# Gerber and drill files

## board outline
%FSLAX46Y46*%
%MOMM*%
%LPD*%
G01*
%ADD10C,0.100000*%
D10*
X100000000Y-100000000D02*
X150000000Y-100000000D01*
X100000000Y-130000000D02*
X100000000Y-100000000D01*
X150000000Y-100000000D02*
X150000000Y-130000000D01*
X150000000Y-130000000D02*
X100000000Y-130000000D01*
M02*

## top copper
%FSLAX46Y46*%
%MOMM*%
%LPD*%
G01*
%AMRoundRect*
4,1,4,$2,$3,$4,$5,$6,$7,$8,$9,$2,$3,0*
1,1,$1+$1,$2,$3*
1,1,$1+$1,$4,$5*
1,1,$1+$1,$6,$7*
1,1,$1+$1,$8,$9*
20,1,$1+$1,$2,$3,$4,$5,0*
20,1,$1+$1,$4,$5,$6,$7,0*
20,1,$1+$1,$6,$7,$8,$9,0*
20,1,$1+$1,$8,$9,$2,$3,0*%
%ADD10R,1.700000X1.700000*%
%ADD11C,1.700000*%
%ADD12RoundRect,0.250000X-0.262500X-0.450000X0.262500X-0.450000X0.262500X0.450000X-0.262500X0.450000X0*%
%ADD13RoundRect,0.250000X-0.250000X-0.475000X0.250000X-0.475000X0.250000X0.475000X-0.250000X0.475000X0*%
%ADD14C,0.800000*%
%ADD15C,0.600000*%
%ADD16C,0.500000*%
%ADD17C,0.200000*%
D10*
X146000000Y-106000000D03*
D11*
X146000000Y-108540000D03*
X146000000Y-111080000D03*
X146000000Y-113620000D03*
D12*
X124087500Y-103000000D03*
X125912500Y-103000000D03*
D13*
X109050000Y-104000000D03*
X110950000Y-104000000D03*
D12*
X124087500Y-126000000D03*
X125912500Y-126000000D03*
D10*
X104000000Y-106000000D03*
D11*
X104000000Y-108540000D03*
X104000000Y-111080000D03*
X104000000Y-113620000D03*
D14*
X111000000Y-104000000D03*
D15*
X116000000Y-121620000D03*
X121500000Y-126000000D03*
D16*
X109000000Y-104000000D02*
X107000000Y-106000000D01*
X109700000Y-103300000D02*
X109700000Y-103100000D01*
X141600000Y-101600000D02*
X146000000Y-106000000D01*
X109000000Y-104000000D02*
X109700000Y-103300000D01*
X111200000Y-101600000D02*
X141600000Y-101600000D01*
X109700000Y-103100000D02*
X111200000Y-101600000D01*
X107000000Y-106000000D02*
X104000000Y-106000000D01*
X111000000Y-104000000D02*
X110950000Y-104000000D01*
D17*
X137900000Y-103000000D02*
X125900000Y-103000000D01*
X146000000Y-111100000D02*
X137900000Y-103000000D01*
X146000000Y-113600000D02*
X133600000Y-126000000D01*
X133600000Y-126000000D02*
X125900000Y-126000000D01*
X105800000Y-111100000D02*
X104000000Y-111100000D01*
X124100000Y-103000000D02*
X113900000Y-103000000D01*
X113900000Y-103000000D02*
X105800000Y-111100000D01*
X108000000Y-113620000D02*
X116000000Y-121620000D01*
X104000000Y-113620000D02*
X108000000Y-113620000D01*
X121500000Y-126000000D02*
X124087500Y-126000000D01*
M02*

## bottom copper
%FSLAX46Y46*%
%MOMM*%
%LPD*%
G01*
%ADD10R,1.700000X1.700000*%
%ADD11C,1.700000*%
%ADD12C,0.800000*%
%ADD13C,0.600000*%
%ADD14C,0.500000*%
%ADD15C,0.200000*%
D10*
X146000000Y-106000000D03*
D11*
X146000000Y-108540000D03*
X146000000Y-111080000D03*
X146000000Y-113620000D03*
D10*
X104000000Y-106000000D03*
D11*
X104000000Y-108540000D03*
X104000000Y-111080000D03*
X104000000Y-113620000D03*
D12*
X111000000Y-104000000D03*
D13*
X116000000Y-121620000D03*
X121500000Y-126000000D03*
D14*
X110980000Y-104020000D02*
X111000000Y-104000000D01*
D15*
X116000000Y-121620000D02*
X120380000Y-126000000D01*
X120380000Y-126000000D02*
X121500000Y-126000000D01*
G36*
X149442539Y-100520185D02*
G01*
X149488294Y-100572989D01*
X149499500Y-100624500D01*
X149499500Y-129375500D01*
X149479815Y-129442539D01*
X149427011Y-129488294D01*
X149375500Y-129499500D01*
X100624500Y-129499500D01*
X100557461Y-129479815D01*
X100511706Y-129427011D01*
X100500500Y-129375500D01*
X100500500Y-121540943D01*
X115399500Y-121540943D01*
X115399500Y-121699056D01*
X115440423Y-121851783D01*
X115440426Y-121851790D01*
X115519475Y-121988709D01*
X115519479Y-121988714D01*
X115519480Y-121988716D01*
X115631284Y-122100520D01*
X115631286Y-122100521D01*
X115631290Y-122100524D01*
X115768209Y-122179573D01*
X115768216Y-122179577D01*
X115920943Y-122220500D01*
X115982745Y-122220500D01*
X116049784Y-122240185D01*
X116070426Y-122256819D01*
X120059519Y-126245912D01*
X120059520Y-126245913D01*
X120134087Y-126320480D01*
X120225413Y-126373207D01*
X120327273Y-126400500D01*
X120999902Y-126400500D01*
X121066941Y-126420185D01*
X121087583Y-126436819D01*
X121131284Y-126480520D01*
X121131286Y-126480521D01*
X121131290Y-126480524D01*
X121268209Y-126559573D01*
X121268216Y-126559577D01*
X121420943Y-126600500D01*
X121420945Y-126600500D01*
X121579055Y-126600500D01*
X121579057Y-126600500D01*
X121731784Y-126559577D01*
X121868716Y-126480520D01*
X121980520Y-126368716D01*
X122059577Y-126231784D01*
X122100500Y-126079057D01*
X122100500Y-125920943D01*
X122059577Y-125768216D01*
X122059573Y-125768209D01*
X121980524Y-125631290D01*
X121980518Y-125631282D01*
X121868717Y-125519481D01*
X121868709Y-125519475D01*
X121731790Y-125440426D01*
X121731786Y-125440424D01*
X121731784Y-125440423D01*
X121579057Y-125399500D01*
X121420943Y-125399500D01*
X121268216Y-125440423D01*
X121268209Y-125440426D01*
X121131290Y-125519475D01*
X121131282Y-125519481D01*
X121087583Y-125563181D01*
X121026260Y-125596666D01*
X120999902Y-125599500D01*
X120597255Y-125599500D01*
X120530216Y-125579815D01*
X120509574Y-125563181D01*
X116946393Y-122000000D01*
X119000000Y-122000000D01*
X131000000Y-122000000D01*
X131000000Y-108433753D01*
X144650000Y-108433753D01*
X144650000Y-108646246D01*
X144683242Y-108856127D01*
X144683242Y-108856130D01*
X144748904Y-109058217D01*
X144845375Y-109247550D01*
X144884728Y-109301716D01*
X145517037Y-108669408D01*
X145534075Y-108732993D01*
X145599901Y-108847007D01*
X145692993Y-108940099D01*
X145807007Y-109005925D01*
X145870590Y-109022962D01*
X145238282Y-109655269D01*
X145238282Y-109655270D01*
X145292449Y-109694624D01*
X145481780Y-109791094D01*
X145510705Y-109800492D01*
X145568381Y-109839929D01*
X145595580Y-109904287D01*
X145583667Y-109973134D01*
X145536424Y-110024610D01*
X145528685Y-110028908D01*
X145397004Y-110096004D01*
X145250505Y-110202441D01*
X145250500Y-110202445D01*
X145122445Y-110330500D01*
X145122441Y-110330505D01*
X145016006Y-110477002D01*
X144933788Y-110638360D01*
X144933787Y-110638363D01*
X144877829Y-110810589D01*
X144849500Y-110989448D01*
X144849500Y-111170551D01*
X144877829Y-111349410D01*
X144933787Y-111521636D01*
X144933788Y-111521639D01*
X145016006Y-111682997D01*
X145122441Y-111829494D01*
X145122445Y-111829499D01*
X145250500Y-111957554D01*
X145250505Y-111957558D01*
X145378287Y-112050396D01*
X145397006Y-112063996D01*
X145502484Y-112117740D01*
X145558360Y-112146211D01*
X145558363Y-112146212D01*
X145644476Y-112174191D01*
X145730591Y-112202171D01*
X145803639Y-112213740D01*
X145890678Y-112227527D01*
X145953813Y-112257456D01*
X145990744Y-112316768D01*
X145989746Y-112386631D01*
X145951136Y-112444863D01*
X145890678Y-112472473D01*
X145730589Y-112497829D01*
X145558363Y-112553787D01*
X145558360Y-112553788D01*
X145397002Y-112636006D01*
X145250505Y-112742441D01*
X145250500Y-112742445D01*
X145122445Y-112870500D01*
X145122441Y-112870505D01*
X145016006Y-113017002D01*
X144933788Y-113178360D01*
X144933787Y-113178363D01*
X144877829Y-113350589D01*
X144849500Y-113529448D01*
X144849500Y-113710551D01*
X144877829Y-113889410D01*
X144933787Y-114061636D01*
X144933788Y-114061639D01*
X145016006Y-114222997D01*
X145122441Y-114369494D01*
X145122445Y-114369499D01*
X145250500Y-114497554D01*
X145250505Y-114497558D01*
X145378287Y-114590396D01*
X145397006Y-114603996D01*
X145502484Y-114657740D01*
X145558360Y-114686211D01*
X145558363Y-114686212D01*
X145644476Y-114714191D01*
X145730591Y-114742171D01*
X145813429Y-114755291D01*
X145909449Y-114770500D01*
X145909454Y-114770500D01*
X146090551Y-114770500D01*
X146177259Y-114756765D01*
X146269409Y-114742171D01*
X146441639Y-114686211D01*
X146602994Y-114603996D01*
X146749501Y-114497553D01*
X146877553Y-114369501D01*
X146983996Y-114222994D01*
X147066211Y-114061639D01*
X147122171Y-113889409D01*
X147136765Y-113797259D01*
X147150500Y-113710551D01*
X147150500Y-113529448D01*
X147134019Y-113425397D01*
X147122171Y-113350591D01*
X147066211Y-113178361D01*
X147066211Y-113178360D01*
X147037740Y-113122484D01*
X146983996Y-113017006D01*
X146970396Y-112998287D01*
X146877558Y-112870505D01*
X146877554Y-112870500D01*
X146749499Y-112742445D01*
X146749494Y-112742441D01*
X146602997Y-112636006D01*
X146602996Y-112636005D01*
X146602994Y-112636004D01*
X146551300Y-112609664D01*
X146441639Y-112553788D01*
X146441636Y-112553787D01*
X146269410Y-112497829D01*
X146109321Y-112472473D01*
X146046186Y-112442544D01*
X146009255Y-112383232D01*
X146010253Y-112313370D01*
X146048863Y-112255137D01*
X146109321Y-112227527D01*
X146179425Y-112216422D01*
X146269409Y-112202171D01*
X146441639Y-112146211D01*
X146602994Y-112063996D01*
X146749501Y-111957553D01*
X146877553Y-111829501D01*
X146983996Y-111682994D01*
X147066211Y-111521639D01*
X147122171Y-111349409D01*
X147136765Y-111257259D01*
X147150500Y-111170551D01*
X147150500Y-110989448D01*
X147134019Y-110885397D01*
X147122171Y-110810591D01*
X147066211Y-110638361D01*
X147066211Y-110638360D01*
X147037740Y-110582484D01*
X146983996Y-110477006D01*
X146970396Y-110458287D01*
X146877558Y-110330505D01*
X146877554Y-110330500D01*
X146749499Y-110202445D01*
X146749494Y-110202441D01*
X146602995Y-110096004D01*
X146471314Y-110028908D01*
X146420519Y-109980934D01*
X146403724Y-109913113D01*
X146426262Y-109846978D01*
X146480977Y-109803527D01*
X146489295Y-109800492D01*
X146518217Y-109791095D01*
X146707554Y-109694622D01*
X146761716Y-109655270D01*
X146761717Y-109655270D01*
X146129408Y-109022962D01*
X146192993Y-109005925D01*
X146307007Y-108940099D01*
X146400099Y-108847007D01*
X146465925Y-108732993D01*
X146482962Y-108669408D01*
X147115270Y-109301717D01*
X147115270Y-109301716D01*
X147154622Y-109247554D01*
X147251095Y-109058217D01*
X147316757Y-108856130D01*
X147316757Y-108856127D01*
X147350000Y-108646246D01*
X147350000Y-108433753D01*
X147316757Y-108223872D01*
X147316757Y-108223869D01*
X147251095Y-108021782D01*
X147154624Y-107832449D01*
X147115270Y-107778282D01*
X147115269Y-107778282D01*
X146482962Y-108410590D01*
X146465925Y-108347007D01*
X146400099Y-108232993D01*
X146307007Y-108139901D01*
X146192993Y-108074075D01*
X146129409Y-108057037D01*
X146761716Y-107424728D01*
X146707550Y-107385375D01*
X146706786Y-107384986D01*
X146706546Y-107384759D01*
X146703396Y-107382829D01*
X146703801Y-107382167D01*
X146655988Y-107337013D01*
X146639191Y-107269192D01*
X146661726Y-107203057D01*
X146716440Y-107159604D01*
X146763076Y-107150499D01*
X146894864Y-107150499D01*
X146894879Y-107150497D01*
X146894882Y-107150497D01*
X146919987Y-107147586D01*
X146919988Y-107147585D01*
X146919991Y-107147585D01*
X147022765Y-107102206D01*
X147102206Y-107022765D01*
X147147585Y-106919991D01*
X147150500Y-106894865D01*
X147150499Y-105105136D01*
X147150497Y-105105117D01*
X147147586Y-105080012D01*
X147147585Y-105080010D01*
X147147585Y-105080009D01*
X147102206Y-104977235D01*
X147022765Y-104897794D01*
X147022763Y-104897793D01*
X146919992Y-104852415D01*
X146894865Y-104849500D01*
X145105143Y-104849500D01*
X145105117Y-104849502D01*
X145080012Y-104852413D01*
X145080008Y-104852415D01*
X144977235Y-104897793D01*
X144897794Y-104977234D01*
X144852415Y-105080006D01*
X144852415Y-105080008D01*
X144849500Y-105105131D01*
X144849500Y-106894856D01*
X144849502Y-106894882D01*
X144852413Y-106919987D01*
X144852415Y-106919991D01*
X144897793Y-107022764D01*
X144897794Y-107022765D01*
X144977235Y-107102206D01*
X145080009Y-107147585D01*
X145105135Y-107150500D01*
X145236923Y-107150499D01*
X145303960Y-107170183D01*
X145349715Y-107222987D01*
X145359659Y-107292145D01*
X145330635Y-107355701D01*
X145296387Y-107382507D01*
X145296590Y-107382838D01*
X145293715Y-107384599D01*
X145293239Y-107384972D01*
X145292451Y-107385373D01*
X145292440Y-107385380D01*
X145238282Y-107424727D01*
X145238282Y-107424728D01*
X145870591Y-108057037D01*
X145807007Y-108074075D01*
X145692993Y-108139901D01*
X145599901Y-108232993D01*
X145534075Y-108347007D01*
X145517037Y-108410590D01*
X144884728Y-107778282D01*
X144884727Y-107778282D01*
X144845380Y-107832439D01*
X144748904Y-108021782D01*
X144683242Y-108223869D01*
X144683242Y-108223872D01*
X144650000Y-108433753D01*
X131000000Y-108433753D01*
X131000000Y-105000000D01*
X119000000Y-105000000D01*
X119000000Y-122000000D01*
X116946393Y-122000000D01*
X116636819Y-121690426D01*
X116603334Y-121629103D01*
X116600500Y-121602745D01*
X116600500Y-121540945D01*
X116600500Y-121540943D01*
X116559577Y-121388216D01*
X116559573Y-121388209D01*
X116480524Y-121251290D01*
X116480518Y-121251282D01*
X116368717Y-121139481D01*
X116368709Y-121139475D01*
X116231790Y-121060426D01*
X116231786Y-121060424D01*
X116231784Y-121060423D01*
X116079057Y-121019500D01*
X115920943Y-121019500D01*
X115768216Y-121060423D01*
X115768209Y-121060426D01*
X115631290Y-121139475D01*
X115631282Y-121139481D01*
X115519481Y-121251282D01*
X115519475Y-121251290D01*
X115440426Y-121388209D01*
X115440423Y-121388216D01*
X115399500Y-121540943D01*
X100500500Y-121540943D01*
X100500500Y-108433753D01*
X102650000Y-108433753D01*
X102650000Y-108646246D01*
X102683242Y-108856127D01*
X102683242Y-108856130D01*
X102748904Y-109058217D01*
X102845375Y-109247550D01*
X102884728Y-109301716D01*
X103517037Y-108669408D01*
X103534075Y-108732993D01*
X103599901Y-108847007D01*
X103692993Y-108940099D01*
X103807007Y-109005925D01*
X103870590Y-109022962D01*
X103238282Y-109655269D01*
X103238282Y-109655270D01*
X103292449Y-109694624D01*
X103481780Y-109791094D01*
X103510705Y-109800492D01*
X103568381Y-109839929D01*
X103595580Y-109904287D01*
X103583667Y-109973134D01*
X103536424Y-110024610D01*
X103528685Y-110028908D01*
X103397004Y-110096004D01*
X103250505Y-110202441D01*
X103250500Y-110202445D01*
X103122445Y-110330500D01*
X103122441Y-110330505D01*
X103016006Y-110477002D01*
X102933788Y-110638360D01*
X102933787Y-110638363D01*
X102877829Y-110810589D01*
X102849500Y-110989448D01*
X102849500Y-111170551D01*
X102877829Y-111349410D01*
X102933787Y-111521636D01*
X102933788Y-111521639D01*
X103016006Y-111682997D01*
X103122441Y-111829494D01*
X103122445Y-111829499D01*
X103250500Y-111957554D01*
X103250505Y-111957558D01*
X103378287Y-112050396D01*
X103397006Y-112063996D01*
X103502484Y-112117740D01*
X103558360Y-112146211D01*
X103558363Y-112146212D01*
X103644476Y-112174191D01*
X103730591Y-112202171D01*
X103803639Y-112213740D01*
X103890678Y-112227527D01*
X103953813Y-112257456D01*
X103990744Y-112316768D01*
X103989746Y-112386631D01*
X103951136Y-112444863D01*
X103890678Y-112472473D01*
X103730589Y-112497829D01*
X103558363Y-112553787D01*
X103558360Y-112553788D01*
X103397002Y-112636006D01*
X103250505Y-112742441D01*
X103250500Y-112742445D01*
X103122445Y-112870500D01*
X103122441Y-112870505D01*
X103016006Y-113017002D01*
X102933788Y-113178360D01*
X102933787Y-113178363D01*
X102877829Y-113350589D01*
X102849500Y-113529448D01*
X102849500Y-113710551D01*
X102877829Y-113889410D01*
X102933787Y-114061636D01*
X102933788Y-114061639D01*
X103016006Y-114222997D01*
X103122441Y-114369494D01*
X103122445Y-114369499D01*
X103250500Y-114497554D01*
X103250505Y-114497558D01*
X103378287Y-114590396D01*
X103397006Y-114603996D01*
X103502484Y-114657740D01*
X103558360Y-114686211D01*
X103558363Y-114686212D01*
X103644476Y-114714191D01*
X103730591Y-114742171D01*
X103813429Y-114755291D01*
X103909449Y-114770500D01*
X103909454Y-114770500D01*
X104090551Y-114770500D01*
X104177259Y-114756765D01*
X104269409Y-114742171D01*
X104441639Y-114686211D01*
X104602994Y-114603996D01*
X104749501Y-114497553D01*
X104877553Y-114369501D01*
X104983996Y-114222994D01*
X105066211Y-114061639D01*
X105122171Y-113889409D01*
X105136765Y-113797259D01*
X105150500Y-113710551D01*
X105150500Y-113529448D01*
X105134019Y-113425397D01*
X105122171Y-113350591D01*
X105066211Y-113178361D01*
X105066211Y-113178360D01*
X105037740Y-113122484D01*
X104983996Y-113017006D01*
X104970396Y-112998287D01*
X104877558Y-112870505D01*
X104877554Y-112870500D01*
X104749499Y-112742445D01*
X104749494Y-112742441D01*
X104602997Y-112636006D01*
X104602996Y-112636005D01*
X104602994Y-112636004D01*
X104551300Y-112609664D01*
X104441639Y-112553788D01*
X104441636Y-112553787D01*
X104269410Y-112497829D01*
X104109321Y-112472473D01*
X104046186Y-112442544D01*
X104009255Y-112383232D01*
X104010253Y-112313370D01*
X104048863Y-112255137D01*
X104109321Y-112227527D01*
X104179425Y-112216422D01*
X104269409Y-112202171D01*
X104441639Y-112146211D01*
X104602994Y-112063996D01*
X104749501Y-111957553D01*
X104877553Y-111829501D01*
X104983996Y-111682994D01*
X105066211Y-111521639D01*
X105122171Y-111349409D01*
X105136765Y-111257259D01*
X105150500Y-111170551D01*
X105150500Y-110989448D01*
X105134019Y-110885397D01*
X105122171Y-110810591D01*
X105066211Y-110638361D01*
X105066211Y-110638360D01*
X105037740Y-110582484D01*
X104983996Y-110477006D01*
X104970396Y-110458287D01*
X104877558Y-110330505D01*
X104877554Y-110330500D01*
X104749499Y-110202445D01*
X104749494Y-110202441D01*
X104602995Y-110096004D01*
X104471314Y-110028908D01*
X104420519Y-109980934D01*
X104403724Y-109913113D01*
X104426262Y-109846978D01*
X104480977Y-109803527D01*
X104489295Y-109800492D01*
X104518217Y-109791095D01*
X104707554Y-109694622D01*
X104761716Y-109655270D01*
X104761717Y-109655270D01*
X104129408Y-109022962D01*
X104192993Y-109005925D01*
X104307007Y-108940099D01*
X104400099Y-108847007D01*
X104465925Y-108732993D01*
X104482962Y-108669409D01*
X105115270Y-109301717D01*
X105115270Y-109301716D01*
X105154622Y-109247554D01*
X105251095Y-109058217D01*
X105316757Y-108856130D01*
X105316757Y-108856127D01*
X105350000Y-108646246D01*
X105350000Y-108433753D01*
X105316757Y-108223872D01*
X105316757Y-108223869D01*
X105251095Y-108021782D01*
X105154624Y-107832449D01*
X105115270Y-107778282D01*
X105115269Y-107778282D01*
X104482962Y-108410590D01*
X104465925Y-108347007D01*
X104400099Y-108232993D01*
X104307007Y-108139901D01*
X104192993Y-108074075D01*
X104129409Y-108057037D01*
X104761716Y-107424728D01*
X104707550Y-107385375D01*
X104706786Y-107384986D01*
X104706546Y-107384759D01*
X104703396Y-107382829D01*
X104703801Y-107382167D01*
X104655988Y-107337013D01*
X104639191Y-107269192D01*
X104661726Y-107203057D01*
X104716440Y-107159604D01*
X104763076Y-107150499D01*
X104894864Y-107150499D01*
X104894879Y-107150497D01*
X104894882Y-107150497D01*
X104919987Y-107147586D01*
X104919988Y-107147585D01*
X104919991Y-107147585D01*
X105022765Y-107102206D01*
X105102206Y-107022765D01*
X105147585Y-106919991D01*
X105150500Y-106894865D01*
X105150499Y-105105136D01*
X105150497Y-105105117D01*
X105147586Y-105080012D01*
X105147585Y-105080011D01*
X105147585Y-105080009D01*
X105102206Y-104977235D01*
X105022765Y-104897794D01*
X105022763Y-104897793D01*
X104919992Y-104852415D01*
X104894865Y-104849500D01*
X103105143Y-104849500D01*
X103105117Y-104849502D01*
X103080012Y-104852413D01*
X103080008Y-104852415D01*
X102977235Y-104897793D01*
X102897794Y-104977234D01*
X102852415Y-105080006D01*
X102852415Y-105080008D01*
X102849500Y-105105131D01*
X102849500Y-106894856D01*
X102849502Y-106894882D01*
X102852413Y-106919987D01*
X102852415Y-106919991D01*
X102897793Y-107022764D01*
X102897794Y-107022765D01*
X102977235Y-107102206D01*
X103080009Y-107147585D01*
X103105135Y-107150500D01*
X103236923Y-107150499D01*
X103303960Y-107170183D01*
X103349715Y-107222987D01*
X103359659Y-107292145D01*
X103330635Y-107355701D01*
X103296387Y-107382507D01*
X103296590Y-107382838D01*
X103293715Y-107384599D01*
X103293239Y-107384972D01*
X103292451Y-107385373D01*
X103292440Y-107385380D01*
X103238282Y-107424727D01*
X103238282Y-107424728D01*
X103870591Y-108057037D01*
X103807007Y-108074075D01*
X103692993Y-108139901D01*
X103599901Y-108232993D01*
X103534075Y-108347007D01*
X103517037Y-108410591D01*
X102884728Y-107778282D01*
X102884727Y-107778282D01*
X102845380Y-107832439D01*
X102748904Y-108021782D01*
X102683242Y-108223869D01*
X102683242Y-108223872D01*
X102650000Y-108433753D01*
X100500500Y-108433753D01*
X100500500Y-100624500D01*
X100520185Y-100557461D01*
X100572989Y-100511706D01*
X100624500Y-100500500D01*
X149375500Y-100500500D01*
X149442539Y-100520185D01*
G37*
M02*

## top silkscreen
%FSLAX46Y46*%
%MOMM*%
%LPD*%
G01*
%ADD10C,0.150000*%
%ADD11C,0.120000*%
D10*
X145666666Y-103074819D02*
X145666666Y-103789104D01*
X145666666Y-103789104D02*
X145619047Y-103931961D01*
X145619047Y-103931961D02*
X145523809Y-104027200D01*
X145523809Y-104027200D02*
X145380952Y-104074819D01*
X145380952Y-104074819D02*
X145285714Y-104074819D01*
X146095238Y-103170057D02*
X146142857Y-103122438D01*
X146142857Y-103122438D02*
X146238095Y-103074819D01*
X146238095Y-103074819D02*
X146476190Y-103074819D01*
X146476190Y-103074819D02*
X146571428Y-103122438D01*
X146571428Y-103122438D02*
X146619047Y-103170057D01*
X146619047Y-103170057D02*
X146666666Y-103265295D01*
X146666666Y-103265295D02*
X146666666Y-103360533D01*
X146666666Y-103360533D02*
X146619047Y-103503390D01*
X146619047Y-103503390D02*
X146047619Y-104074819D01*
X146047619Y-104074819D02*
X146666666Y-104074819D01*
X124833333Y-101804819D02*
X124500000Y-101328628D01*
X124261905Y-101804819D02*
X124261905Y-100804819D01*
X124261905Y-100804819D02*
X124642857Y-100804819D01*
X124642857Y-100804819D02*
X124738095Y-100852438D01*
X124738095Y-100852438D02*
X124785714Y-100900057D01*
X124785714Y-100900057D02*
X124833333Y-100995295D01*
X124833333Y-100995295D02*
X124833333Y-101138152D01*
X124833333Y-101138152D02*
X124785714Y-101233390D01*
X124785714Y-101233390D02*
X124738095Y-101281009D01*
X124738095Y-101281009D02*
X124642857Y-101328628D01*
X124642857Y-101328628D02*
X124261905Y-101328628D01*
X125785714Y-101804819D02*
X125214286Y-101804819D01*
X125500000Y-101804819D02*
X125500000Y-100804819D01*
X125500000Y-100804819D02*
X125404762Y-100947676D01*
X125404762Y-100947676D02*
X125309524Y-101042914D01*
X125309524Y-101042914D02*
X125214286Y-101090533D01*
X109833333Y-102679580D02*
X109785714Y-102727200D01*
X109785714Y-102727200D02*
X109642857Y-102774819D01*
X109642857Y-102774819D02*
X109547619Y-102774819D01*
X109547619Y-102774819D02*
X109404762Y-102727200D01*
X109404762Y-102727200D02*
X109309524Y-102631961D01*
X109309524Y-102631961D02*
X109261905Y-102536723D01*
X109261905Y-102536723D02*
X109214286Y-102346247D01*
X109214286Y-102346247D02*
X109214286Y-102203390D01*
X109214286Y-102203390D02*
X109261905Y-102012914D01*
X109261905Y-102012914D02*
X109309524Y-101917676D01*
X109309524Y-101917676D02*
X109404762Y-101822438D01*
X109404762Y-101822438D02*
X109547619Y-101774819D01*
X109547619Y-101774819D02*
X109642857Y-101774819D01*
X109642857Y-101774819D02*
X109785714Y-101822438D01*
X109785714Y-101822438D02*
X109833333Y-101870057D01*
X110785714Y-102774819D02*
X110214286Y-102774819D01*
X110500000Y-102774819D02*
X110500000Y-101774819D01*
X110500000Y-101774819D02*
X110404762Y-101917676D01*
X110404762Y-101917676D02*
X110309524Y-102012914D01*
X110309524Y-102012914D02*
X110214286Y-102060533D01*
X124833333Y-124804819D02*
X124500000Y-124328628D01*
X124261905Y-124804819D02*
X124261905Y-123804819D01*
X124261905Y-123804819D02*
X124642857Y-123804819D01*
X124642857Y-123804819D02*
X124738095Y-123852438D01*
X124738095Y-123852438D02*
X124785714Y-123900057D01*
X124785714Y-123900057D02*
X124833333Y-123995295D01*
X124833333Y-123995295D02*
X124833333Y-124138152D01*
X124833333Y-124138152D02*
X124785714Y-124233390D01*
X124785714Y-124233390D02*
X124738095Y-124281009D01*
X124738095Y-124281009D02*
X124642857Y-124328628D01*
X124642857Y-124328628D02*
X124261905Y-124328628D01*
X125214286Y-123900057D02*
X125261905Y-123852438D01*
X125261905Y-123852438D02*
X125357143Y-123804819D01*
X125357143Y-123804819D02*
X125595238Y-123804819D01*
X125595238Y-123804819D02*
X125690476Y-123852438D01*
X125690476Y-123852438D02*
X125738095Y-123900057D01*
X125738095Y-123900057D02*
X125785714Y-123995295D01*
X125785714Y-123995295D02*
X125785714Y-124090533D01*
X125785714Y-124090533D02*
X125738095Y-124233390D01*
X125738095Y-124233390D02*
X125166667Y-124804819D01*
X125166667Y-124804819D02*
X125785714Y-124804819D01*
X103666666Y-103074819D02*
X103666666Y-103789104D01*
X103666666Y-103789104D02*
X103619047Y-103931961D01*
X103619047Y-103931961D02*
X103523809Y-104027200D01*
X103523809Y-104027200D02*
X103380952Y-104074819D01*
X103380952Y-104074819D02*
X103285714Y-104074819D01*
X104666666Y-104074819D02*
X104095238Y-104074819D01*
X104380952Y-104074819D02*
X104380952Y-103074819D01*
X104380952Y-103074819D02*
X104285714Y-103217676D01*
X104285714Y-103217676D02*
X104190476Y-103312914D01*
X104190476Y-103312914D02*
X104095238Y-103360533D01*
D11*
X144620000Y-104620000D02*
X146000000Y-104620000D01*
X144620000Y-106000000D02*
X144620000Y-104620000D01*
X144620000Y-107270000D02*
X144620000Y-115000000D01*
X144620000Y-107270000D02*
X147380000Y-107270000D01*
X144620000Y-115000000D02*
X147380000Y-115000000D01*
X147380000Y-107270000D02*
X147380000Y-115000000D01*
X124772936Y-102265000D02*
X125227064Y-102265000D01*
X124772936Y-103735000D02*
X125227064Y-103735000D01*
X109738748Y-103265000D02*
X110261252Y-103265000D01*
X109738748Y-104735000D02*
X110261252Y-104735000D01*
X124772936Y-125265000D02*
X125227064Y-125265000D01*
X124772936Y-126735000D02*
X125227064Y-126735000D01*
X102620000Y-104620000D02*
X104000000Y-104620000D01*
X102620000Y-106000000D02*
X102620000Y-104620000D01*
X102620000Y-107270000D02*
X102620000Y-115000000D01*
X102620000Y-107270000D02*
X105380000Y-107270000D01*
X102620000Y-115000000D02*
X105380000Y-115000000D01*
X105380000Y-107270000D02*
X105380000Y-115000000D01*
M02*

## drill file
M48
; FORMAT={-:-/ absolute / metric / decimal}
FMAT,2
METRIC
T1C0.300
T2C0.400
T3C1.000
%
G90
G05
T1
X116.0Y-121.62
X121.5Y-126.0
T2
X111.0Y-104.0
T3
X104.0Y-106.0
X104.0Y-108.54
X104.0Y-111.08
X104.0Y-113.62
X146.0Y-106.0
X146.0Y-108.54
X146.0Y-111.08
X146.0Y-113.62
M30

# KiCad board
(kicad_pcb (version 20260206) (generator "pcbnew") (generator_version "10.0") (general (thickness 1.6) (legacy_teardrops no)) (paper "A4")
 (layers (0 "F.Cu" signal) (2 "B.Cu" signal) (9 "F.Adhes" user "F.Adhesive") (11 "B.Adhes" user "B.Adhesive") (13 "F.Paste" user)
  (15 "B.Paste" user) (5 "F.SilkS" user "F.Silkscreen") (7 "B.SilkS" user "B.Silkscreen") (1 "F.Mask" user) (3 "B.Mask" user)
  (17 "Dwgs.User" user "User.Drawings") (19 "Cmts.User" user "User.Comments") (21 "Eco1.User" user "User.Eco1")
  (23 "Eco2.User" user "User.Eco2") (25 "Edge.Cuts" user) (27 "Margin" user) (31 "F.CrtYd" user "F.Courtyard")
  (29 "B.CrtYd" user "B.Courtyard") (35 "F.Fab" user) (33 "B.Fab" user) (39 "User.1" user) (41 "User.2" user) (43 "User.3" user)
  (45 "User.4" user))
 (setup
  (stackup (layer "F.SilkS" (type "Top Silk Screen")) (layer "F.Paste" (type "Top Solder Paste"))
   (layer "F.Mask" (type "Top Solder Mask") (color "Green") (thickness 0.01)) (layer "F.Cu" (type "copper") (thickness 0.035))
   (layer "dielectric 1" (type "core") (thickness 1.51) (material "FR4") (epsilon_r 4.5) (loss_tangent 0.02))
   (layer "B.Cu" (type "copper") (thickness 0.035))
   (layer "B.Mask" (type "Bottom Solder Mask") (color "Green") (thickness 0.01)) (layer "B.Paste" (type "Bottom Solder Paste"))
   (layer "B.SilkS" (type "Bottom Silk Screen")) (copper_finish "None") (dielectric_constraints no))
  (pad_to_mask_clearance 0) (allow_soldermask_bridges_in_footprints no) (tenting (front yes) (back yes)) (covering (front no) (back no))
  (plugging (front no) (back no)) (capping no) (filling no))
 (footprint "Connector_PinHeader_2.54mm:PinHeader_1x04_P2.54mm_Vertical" (layer "F.Cu") (at 146 106)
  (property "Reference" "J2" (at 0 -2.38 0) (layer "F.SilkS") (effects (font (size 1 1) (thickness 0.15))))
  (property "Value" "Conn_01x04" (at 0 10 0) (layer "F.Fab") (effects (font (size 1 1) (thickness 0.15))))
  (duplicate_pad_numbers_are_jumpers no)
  (fp_line (start -1.38 -1.38) (end 0 -1.38) (stroke (width 0.12) (type solid)) (layer "F.SilkS"))
  (fp_line (start -1.38 0) (end -1.38 -1.38) (stroke (width 0.12) (type solid)) (layer "F.SilkS"))
  (fp_line (start -1.38 1.27) (end -1.38 9) (stroke (width 0.12) (type solid)) (layer "F.SilkS"))
  (fp_line (start -1.38 1.27) (end 1.38 1.27) (stroke (width 0.12) (type solid)) (layer "F.SilkS"))
  (fp_line (start -1.38 9) (end 1.38 9) (stroke (width 0.12) (type solid)) (layer "F.SilkS"))
  (fp_line (start 1.38 1.27) (end 1.38 9) (stroke (width 0.12) (type solid)) (layer "F.SilkS"))
  (pad "1" thru_hole rect (at 0 0) (size 1.7 1.7) (drill 1) (layers "*.Cu" "*.Mask") (remove_unused_layers no) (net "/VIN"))
  (pad "2" thru_hole circle (at 0 2.54) (size 1.7 1.7) (drill 1) (layers "*.Cu" "*.Mask") (remove_unused_layers no) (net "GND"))
  (pad "3" thru_hole circle (at 0 5.08) (size 1.7 1.7) (drill 1) (layers "*.Cu" "*.Mask") (remove_unused_layers no) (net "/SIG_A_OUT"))
  (pad "4" thru_hole circle (at 0 7.62) (size 1.7 1.7) (drill 1) (layers "*.Cu" "*.Mask") (remove_unused_layers no) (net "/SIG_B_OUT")))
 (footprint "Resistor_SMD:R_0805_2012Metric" (layer "F.Cu") (at 125 103)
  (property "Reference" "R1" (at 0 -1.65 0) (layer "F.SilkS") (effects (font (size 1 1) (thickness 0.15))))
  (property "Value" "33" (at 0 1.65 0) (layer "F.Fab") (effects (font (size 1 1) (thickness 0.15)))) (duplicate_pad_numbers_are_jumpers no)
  (fp_line (start -0.227064 -0.735) (end 0.227064 -0.735) (stroke (width 0.12) (type solid)) (layer "F.SilkS"))
  (fp_line (start -0.227064 0.735) (end 0.227064 0.735) (stroke (width 0.12) (type solid)) (layer "F.SilkS"))
  (pad "1" smd roundrect (at -0.9125 0) (size 1.025 1.4) (layers "F.Cu" "F.Mask" "F.Paste") (roundrect_rratio 0.243902) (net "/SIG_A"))
  (pad "2" smd roundrect (at 0.9125 0) (size 1.025 1.4) (layers "F.Cu" "F.Mask" "F.Paste") (roundrect_rratio 0.243902) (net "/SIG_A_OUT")))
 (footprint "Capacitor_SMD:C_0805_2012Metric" (layer "F.Cu") (at 110 104)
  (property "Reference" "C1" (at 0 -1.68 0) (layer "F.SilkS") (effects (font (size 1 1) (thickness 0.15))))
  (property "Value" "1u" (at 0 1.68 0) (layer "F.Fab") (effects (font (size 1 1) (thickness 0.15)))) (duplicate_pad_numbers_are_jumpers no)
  (fp_line (start -0.261252 -0.735) (end 0.261252 -0.735) (stroke (width 0.12) (type solid)) (layer "F.SilkS"))
  (fp_line (start -0.261252 0.735) (end 0.261252 0.735) (stroke (width 0.12) (type solid)) (layer "F.SilkS"))
  (pad "1" smd roundrect (at -0.95 0) (size 1 1.45) (layers "F.Cu" "F.Mask" "F.Paste") (roundrect_rratio 0.25) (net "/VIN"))
  (pad "2" smd roundrect (at 0.95 0) (size 1 1.45) (layers "F.Cu" "F.Mask" "F.Paste") (roundrect_rratio 0.25) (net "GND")))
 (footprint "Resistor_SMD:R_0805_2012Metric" (layer "F.Cu") (at 125 126)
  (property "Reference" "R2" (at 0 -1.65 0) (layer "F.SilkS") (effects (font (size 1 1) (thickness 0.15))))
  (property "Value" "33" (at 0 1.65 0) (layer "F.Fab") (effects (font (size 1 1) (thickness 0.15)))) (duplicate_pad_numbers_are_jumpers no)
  (fp_line (start -0.227064 -0.735) (end 0.227064 -0.735) (stroke (width 0.12) (type solid)) (layer "F.SilkS"))
  (fp_line (start -0.227064 0.735) (end 0.227064 0.735) (stroke (width 0.12) (type solid)) (layer "F.SilkS"))
  (pad "1" smd roundrect (at -0.9125 0) (size 1.025 1.4) (layers "F.Cu" "F.Mask" "F.Paste") (roundrect_rratio 0.243902) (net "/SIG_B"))
  (pad "2" smd roundrect (at 0.9125 0) (size 1.025 1.4) (layers "F.Cu" "F.Mask" "F.Paste") (roundrect_rratio 0.243902) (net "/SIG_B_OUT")))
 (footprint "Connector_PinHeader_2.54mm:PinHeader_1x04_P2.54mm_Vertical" (layer "F.Cu") (at 104 106)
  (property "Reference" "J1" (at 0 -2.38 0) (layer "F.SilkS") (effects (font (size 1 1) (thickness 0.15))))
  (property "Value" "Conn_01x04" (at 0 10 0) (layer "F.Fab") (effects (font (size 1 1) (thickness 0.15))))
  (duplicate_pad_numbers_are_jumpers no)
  (fp_line (start -1.38 -1.38) (end 0 -1.38) (stroke (width 0.12) (type solid)) (layer "F.SilkS"))
  (fp_line (start -1.38 0) (end -1.38 -1.38) (stroke (width 0.12) (type solid)) (layer "F.SilkS"))
  (fp_line (start -1.38 1.27) (end -1.38 9) (stroke (width 0.12) (type solid)) (layer "F.SilkS"))
  (fp_line (start -1.38 1.27) (end 1.38 1.27) (stroke (width 0.12) (type solid)) (layer "F.SilkS"))
  (fp_line (start -1.38 9) (end 1.38 9) (stroke (width 0.12) (type solid)) (layer "F.SilkS"))
  (fp_line (start 1.38 1.27) (end 1.38 9) (stroke (width 0.12) (type solid)) (layer "F.SilkS"))
  (pad "1" thru_hole rect (at 0 0) (size 1.7 1.7) (drill 1) (layers "*.Cu" "*.Mask") (remove_unused_layers no) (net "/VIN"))
  (pad "2" thru_hole circle (at 0 2.54) (size 1.7 1.7) (drill 1) (layers "*.Cu" "*.Mask") (remove_unused_layers no) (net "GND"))
  (pad "3" thru_hole circle (at 0 5.08) (size 1.7 1.7) (drill 1) (layers "*.Cu" "*.Mask") (remove_unused_layers no) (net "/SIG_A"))
  (pad "4" thru_hole circle (at 0 7.62) (size 1.7 1.7) (drill 1) (layers "*.Cu" "*.Mask") (remove_unused_layers no) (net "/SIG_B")))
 (gr_line (start 100 100) (end 150 100) (stroke (width 0.1) (type default)) (layer "Edge.Cuts"))
 (gr_line (start 100 130) (end 100 100) (stroke (width 0.1) (type default)) (layer "Edge.Cuts"))
 (gr_line (start 150 100) (end 150 130) (stroke (width 0.1) (type default)) (layer "Edge.Cuts"))
 (gr_line (start 150 130) (end 100 130) (stroke (width 0.1) (type default)) (layer "Edge.Cuts"))
 (segment (start 109 104) (end 107 106) (width 0.5) (layer "F.Cu") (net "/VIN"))
 (segment (start 109.7 103.3) (end 109.7 103.1) (width 0.5) (layer "F.Cu") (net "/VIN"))
 (segment (start 141.6 101.6) (end 146 106) (width 0.5) (layer "F.Cu") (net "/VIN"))
 (segment (start 109 104) (end 109.7 103.3) (width 0.5) (layer "F.Cu") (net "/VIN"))
 (segment (start 111.2 101.6) (end 141.6 101.6) (width 0.5) (layer "F.Cu") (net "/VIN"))
 (segment (start 109.7 103.1) (end 111.2 101.6) (width 0.5) (layer "F.Cu") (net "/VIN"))
 (segment (start 107 106) (end 104 106) (width 0.5) (layer "F.Cu") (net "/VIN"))
 (segment (start 111 104) (end 110.95 104) (width 0.5) (layer "F.Cu") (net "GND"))
 (via (at 111 104) (size 0.8) (drill 0.4) (layers "F.Cu" "B.Cu") (capping yes) (filling yes) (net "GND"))
 (segment (start 110.98 104.02) (end 111 104) (width 0.5) (layer "B.Cu") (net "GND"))
 (segment (start 137.9 103) (end 125.9 103) (width 0.2) (layer "F.Cu") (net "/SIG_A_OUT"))
 (segment (start 146 111.1) (end 137.9 103) (width 0.2) (layer "F.Cu") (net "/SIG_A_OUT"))
 (segment (start 146 113.6) (end 133.6 126) (width 0.2) (layer "F.Cu") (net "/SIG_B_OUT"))
 (segment (start 133.6 126) (end 125.9 126) (width 0.2) (layer "F.Cu") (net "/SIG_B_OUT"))
 (segment (start 105.8 111.1) (end 104 111.1) (width 0.2) (layer "F.Cu") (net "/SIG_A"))
 (segment (start 124.1 103) (end 113.9 103) (width 0.2) (layer "F.Cu") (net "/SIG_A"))
 (segment (start 113.9 103) (end 105.8 111.1) (width 0.2) (layer "F.Cu") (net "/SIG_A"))
 (segment (start 108 113.62) (end 116 121.62) (width 0.2) (locked yes) (layer "F.Cu") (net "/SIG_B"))
 (segment (start 104 113.62) (end 108 113.62) (width 0.2) (locked yes) (layer "F.Cu") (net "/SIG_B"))
 (segment (start 121.5 126) (end 124.0875 126) (width 0.2) (locked yes) (layer "F.Cu") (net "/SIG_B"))
 (via (at 116 121.62) (size 0.6) (drill 0.3) (layers "F.Cu" "B.Cu") (locked yes) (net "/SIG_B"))
 (via (at 121.5 126) (size 0.6) (drill 0.3) (layers "F.Cu" "B.Cu") (locked yes) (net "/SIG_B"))
 (segment (start 116 121.62) (end 120.38 126) (width 0.2) (locked yes) (layer "B.Cu") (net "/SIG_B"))
 (segment (start 120.38 126) (end 121.5 126) (width 0.2) (locked yes) (layer "B.Cu") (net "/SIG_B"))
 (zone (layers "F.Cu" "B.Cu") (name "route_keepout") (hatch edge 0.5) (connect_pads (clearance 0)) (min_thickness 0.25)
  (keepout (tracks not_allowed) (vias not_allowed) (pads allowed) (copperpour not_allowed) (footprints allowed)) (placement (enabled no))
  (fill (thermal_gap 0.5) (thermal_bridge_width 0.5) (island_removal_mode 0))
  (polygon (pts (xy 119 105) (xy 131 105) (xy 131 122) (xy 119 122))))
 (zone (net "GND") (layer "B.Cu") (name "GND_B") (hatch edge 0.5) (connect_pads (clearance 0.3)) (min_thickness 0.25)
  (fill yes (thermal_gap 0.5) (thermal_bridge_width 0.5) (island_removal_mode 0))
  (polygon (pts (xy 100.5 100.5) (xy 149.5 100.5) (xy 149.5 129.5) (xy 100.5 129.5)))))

